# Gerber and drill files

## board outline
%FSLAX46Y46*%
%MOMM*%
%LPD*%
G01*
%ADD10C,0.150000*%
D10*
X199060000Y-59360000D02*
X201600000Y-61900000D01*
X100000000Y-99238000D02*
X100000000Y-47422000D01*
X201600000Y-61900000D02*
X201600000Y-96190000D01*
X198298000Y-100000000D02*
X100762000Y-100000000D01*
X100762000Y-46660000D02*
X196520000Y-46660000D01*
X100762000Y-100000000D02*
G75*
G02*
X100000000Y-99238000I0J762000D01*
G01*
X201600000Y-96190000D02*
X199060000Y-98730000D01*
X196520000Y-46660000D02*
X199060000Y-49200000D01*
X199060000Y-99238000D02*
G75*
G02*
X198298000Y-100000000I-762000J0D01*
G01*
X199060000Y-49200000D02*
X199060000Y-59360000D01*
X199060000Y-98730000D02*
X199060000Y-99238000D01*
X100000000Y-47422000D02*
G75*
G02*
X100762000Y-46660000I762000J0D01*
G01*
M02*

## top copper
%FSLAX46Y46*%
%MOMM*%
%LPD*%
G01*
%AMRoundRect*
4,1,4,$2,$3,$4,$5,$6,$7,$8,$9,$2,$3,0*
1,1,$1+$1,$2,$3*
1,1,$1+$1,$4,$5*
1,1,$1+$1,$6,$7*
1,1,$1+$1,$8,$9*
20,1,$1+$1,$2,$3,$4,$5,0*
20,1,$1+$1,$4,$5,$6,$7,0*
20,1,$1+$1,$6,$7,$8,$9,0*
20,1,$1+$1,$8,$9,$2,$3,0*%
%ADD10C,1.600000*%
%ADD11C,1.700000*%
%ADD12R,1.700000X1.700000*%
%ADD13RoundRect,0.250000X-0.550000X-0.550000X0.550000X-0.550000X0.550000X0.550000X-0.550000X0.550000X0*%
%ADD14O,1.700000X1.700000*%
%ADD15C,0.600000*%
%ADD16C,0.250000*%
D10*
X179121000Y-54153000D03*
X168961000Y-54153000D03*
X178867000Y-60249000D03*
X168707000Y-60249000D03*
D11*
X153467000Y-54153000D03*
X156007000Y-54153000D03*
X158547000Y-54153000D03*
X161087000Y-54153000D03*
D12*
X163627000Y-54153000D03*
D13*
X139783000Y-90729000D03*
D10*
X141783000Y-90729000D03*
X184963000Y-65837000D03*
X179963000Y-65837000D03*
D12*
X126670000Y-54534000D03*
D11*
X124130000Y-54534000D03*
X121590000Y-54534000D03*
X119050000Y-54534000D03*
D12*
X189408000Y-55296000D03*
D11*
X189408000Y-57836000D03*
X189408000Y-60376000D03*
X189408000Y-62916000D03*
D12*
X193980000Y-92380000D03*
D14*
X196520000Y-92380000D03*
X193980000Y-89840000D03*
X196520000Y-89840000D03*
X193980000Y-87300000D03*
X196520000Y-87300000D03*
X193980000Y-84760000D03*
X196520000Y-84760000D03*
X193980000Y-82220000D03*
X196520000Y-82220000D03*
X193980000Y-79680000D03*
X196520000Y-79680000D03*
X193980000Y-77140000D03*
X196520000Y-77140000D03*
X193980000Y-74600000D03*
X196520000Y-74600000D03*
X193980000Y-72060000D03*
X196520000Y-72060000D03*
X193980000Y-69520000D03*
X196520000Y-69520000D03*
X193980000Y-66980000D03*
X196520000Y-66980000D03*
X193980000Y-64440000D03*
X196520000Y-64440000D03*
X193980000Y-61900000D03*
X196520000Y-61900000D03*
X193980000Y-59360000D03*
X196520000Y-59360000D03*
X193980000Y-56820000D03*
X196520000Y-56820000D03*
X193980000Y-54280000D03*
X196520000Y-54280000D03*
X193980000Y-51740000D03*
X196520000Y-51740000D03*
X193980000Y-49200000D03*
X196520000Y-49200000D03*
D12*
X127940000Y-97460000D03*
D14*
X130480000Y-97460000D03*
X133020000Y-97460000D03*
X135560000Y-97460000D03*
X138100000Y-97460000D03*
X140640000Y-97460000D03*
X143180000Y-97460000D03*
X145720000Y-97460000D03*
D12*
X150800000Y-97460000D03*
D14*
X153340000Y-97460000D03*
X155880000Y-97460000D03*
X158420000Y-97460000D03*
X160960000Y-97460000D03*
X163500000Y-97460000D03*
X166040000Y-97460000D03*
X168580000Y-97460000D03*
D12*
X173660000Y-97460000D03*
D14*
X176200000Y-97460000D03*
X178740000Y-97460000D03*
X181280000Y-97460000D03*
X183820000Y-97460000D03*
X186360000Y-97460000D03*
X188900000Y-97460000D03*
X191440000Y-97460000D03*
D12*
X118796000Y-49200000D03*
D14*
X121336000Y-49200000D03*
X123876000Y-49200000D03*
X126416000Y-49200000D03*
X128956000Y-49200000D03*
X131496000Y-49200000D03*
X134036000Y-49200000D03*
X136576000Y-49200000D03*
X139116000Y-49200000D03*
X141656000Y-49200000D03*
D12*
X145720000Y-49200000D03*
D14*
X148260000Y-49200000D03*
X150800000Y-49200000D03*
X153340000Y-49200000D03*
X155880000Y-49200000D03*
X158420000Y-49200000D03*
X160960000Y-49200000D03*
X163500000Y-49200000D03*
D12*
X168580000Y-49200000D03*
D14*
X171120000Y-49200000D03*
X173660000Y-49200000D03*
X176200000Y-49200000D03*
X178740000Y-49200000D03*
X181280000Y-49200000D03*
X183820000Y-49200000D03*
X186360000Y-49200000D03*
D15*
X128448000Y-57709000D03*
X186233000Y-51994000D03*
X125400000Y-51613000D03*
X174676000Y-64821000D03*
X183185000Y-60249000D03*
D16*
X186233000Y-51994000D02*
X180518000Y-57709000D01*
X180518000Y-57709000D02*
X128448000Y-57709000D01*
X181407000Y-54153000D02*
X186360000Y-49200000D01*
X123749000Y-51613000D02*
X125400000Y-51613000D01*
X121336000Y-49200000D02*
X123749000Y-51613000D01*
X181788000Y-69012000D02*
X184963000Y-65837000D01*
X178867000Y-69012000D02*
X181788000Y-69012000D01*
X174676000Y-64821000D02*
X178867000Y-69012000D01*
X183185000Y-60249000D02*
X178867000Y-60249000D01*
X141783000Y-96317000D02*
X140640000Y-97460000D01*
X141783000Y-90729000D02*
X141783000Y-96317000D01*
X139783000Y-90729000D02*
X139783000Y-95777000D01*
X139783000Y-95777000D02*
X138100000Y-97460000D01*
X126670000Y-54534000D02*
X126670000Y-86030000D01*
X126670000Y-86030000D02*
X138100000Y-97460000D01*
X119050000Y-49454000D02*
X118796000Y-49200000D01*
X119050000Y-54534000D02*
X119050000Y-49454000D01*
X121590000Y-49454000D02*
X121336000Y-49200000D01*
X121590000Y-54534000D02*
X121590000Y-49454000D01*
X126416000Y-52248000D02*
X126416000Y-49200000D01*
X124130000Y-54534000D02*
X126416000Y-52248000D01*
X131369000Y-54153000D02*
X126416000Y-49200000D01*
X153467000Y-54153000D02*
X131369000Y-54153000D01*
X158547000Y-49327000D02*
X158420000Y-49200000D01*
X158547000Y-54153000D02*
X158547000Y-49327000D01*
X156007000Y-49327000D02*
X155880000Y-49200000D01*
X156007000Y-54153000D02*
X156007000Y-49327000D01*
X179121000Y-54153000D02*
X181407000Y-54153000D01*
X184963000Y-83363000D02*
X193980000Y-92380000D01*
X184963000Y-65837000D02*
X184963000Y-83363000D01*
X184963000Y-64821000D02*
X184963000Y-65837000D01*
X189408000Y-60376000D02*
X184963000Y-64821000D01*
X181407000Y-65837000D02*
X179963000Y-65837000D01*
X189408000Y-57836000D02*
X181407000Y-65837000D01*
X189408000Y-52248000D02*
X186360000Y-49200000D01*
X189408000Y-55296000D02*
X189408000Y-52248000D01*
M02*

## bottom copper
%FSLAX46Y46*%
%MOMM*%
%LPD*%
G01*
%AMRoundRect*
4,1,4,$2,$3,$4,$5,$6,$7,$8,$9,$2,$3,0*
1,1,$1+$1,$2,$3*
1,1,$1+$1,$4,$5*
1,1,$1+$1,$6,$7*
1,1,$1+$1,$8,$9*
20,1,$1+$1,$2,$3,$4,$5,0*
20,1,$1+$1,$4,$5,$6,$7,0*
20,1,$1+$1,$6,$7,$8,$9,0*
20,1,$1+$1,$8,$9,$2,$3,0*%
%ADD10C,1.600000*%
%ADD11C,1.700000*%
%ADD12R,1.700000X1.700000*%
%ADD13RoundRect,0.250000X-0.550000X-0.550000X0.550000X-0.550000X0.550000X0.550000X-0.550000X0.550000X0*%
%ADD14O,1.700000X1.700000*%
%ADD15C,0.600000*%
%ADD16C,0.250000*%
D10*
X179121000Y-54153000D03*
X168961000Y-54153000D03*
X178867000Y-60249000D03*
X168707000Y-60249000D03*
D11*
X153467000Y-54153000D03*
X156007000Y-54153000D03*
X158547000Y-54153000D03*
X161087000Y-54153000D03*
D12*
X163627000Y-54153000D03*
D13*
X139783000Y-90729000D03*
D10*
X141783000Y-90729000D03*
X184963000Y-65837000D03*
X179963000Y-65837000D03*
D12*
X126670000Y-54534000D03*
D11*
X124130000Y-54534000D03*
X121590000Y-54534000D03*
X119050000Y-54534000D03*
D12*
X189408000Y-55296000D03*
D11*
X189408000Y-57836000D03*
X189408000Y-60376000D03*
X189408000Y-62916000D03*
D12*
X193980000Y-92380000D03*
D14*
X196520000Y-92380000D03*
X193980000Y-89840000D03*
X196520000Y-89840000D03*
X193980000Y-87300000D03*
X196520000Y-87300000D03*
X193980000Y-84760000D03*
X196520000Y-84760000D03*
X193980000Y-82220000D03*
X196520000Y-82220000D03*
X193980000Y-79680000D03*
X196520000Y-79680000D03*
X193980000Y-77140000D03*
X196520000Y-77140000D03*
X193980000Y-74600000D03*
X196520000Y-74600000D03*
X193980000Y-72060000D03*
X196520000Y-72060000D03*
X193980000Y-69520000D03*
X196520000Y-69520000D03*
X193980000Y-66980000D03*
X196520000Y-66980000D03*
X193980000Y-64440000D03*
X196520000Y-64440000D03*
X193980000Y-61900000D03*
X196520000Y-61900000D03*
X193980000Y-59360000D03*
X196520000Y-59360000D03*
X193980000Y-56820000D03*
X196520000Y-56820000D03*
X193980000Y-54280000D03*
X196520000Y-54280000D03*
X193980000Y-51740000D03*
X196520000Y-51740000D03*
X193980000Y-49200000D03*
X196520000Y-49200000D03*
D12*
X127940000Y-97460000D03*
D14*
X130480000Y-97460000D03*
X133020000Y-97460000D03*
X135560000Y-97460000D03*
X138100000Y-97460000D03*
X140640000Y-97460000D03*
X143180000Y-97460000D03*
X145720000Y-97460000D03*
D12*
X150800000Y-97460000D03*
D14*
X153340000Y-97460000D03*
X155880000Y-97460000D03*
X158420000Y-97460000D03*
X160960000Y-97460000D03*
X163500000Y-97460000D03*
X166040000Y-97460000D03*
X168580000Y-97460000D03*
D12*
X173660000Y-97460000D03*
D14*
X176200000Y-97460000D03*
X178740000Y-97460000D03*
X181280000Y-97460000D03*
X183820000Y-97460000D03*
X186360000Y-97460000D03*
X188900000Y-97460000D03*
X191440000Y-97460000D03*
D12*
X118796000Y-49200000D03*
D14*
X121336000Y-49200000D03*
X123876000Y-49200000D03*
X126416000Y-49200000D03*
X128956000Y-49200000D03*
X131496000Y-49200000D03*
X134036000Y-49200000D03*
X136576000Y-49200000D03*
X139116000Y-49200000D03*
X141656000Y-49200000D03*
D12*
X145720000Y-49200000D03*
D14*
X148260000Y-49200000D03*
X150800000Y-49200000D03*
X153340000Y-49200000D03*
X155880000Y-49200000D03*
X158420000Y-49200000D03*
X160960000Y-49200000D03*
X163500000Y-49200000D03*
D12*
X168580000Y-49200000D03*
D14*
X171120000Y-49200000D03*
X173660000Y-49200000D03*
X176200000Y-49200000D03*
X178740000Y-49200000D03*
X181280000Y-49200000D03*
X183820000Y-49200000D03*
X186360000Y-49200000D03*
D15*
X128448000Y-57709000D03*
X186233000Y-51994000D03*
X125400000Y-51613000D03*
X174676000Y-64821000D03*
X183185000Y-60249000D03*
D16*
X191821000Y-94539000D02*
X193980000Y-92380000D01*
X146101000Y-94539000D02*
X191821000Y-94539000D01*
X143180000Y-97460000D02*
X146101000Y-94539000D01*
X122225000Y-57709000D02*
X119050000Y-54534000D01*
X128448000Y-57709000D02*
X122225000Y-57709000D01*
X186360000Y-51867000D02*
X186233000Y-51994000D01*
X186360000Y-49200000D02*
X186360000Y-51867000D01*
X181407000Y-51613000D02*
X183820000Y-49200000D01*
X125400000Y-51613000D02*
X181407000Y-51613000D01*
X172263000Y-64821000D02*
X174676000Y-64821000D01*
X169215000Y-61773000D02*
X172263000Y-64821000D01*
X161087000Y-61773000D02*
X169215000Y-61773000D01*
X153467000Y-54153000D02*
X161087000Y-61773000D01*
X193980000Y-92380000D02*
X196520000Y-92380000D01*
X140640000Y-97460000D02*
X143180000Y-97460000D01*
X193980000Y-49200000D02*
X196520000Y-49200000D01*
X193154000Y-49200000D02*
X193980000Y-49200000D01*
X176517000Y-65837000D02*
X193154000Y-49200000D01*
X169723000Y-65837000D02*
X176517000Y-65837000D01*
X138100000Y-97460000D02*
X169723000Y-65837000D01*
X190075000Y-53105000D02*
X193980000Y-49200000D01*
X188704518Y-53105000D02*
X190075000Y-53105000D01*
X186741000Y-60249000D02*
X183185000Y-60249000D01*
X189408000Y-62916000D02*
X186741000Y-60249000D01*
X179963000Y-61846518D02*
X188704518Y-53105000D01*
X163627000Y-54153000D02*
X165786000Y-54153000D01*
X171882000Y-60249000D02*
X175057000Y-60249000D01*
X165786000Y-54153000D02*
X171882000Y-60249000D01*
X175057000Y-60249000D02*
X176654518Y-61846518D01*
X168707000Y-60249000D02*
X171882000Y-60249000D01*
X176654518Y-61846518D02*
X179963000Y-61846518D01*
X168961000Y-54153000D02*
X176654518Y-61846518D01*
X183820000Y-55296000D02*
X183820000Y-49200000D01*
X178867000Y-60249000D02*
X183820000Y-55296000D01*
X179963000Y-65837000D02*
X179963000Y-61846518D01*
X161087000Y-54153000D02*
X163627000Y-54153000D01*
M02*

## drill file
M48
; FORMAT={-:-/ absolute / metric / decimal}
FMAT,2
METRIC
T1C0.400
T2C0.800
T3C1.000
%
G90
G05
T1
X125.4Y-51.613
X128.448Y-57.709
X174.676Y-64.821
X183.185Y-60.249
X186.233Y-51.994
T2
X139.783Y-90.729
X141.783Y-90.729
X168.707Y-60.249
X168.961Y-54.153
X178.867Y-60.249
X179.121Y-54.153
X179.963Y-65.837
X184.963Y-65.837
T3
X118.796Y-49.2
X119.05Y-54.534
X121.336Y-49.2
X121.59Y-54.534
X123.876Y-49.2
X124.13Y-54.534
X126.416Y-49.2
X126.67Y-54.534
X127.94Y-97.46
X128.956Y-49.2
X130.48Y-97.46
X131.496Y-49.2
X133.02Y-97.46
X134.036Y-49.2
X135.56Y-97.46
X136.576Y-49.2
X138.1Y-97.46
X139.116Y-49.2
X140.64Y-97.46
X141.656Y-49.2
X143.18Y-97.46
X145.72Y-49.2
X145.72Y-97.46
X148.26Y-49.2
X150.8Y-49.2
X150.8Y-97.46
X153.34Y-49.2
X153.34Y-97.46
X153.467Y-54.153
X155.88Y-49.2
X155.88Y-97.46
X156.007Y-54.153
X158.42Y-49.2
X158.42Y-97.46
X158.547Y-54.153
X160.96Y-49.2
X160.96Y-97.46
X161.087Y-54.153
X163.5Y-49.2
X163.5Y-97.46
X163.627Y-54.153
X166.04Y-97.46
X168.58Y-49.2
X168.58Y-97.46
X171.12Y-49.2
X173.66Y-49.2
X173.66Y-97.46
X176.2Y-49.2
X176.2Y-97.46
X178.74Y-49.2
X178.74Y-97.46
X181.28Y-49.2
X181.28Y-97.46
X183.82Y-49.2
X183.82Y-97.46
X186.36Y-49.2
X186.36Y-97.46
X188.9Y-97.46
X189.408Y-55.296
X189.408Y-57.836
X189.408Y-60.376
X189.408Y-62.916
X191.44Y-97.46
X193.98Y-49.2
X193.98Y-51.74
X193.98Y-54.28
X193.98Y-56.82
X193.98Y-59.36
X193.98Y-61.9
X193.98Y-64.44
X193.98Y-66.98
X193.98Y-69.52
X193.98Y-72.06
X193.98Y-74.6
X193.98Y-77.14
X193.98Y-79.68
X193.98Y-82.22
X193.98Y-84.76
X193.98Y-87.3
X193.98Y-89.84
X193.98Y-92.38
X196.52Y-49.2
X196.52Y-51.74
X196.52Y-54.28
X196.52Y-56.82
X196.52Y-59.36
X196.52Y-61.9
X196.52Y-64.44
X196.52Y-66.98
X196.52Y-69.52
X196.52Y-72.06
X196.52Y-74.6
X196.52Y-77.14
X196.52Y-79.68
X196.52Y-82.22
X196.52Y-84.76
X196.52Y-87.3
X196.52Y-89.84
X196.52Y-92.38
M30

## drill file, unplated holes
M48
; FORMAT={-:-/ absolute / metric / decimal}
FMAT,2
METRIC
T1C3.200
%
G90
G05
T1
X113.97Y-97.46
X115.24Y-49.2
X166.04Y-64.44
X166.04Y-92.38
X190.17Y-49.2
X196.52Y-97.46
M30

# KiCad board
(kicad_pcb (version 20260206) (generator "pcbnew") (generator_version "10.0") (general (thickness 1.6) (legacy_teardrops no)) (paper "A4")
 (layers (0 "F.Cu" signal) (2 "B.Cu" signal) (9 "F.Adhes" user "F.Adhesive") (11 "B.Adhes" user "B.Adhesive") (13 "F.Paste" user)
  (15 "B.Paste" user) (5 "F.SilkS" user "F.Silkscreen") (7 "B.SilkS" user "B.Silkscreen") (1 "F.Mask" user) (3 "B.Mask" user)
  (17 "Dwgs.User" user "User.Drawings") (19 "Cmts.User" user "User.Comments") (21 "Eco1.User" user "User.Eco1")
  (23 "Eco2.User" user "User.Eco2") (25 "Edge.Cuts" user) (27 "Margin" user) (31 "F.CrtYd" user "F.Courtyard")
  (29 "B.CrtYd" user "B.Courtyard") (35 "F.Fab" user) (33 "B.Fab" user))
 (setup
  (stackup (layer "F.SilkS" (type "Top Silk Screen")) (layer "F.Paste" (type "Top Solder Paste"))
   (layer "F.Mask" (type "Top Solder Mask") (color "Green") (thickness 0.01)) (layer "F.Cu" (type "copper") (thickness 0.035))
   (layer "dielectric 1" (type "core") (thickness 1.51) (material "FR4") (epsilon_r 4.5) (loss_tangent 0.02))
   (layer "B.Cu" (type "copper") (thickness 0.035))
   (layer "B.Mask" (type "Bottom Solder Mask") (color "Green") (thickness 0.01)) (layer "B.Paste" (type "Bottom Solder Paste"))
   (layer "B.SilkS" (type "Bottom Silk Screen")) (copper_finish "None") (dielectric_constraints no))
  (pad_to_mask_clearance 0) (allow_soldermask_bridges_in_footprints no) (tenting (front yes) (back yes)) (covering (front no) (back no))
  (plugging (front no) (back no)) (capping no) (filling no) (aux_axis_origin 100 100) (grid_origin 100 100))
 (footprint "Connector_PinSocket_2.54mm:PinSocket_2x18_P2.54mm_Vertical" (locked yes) (layer "F.Cu") (at 193.98 92.38 180)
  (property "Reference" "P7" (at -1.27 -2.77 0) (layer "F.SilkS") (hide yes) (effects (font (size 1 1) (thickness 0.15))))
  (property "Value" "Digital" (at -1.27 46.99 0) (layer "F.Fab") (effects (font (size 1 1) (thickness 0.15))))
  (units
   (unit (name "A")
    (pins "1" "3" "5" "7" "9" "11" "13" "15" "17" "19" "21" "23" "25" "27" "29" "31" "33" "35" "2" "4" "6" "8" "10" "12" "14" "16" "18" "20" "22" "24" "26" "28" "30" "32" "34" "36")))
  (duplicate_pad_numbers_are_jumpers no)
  (pad "1" thru_hole rect (at 0 0 180) (size 1.7 1.7) (drill 1) (layers "*.Cu" "*.Mask") (remove_unused_layers no) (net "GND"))
  (pad "2" thru_hole oval (at -2.54 0 180) (size 1.7 1.7) (drill 1) (layers "*.Cu" "*.Mask") (remove_unused_layers no) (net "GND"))
  (pad "3" thru_hole oval (at 0 2.54 180) (size 1.7 1.7) (drill 1) (layers "*.Cu" "*.Mask") (remove_unused_layers no) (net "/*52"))
  (pad "4" thru_hole oval (at -2.54 2.54 180) (size 1.7 1.7) (drill 1) (layers "*.Cu" "*.Mask") (remove_unused_layers no) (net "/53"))
  (pad "5" thru_hole oval (at 0 5.08 180) (size 1.7 1.7) (drill 1) (layers "*.Cu" "*.Mask") (remove_unused_layers no) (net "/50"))
  (pad "6" thru_hole oval (at -2.54 5.08 180) (size 1.7 1.7) (drill 1) (layers "*.Cu" "*.Mask") (remove_unused_layers no) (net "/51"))
  (pad "7" thru_hole oval (at 0 7.62 180) (size 1.7 1.7) (drill 1) (layers "*.Cu" "*.Mask") (remove_unused_layers no) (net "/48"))
  (pad "8" thru_hole oval (at -2.54 7.62 180) (size 1.7 1.7) (drill 1) (layers "*.Cu" "*.Mask") (remove_unused_layers no) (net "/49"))
  (pad "9" thru_hole oval (at 0 10.16 180) (size 1.7 1.7) (drill 1) (layers "*.Cu" "*.Mask") (remove_unused_layers no) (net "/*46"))
  (pad "10" thru_hole oval (at -2.54 10.16 180) (size 1.7 1.7) (drill 1) (layers "*.Cu" "*.Mask") (remove_unused_layers no) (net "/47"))
  (pad "11" thru_hole oval (at 0 12.7 180) (size 1.7 1.7) (drill 1) (layers "*.Cu" "*.Mask") (remove_unused_layers no) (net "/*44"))
  (pad "12" thru_hole oval (at -2.54 12.7 180) (size 1.7 1.7) (drill 1) (layers "*.Cu" "*.Mask") (remove_unused_layers no) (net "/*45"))
  (pad "13" thru_hole oval (at 0 15.24 180) (size 1.7 1.7) (drill 1) (layers "*.Cu" "*.Mask") (remove_unused_layers no) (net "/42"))
  (pad "14" thru_hole oval (at -2.54 15.24 180) (size 1.7 1.7) (drill 1) (layers "*.Cu" "*.Mask") (remove_unused_layers no) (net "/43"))
  (pad "15" thru_hole oval (at 0 17.78 180) (size 1.7 1.7) (drill 1) (layers "*.Cu" "*.Mask") (remove_unused_layers no) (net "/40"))
  (pad "16" thru_hole oval (at -2.54 17.78 180) (size 1.7 1.7) (drill 1) (layers "*.Cu" "*.Mask") (remove_unused_layers no) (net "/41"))
  (pad "17" thru_hole oval (at 0 20.32 180) (size 1.7 1.7) (drill 1) (layers "*.Cu" "*.Mask") (remove_unused_layers no) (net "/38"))
  (pad "18" thru_hole oval (at -2.54 20.32 180) (size 1.7 1.7) (drill 1) (layers "*.Cu" "*.Mask") (remove_unused_layers no) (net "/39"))
  (pad "19" thru_hole oval (at 0 22.86 180) (size 1.7 1.7) (drill 1) (layers "*.Cu" "*.Mask") (remove_unused_layers no) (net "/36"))
  (pad "20" thru_hole oval (at -2.54 22.86 180) (size 1.7 1.7) (drill 1) (layers "*.Cu" "*.Mask") (remove_unused_layers no) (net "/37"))
  (pad "21" thru_hole oval (at 0 25.4 180) (size 1.7 1.7) (drill 1) (layers "*.Cu" "*.Mask") (remove_unused_layers no) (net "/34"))
  (pad "22" thru_hole oval (at -2.54 25.4 180) (size 1.7 1.7) (drill 1) (layers "*.Cu" "*.Mask") (remove_unused_layers no) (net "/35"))
  (pad "23" thru_hole oval (at 0 27.94 180) (size 1.7 1.7) (drill 1) (layers "*.Cu" "*.Mask") (remove_unused_layers no) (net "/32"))
  (pad "24" thru_hole oval (at -2.54 27.94 180) (size 1.7 1.7) (drill 1) (layers "*.Cu" "*.Mask") (remove_unused_layers no) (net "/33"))
  (pad "25" thru_hole oval (at 0 30.48 180) (size 1.7 1.7) (drill 1) (layers "*.Cu" "*.Mask") (remove_unused_layers no) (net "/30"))
  (pad "26" thru_hole oval (at -2.54 30.48 180) (size 1.7 1.7) (drill 1) (layers "*.Cu" "*.Mask") (remove_unused_layers no) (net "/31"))
  (pad "27" thru_hole oval (at 0 33.02 180) (size 1.7 1.7) (drill 1) (layers "*.Cu" "*.Mask") (remove_unused_layers no) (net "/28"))
  (pad "28" thru_hole oval (at -2.54 33.02 180) (size 1.7 1.7) (drill 1) (layers "*.Cu" "*.Mask") (remove_unused_layers no) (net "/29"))
  (pad "29" thru_hole oval (at 0 35.56 180) (size 1.7 1.7) (drill 1) (layers "*.Cu" "*.Mask") (remove_unused_layers no) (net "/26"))
  (pad "30" thru_hole oval (at -2.54 35.56 180) (size 1.7 1.7) (drill 1) (layers "*.Cu" "*.Mask") (remove_unused_layers no) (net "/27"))
  (pad "31" thru_hole oval (at 0 38.1 180) (size 1.7 1.7) (drill 1) (layers "*.Cu" "*.Mask") (remove_unused_layers no) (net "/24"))
  (pad "32" thru_hole oval (at -2.54 38.1 180) (size 1.7 1.7) (drill 1) (layers "*.Cu" "*.Mask") (remove_unused_layers no) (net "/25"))
  (pad "33" thru_hole oval (at 0 40.64 180) (size 1.7 1.7) (drill 1) (layers "*.Cu" "*.Mask") (remove_unused_layers no) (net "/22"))
  (pad "34" thru_hole oval (at -2.54 40.64 180) (size 1.7 1.7) (drill 1) (layers "*.Cu" "*.Mask") (remove_unused_layers no) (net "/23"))
  (pad "35" thru_hole oval (at 0 43.18 180) (size 1.7 1.7) (drill 1) (layers "*.Cu" "*.Mask") (remove_unused_layers no) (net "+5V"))
  (pad "36" thru_hole oval (at -2.54 43.18 180) (size 1.7 1.7) (drill 1) (layers "*.Cu" "*.Mask") (remove_unused_layers no) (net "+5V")))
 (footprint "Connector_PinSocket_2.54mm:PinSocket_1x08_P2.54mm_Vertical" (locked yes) (layer "F.Cu") (at 127.94 97.46 90)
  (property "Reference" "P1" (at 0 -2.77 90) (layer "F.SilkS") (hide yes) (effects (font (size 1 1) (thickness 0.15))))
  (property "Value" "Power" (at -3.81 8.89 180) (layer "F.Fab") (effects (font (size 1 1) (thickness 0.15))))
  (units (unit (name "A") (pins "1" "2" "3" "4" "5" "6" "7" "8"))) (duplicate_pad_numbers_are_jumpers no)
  (pad "1" thru_hole rect (at 0 0 90) (size 1.7 1.7) (drill 1) (layers "*.Cu" "*.Mask") (remove_unused_layers no)
   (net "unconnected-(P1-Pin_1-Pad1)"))
  (pad "2" thru_hole oval (at 0 2.54 90) (size 1.7 1.7) (drill 1) (layers "*.Cu" "*.Mask") (remove_unused_layers no) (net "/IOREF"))
  (pad "3" thru_hole oval (at 0 5.08 90) (size 1.7 1.7) (drill 1) (layers "*.Cu" "*.Mask") (remove_unused_layers no) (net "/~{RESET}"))
  (pad "4" thru_hole oval (at 0 7.62 90) (size 1.7 1.7) (drill 1) (layers "*.Cu" "*.Mask") (remove_unused_layers no) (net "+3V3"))
  (pad "5" thru_hole oval (at 0 10.16 90) (size 1.7 1.7) (drill 1) (layers "*.Cu" "*.Mask") (remove_unused_layers no) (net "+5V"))
  (pad "6" thru_hole oval (at 0 12.7 90) (size 1.7 1.7) (drill 1) (layers "*.Cu" "*.Mask") (remove_unused_layers no) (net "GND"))
  (pad "7" thru_hole oval (at 0 15.24 90) (size 1.7 1.7) (drill 1) (layers "*.Cu" "*.Mask") (remove_unused_layers no) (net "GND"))
  (pad "8" thru_hole oval (at 0 17.78 90) (size 1.7 1.7) (drill 1) (layers "*.Cu" "*.Mask") (remove_unused_layers no) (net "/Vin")))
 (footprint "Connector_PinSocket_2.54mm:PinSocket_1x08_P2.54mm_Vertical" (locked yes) (layer "F.Cu") (at 150.8 97.46 90)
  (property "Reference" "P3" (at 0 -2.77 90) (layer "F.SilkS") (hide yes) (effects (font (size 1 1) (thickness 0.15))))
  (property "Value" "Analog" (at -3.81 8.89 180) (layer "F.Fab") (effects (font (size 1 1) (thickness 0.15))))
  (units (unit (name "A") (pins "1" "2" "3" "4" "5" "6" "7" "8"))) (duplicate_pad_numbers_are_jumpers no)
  (pad "1" thru_hole rect (at 0 0 90) (size 1.7 1.7) (drill 1) (layers "*.Cu" "*.Mask") (remove_unused_layers no) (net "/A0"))
  (pad "2" thru_hole oval (at 0 2.54 90) (size 1.7 1.7) (drill 1) (layers "*.Cu" "*.Mask") (remove_unused_layers no) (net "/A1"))
  (pad "3" thru_hole oval (at 0 5.08 90) (size 1.7 1.7) (drill 1) (layers "*.Cu" "*.Mask") (remove_unused_layers no) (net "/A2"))
  (pad "4" thru_hole oval (at 0 7.62 90) (size 1.7 1.7) (drill 1) (layers "*.Cu" "*.Mask") (remove_unused_layers no) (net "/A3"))
  (pad "5" thru_hole oval (at 0 10.16 90) (size 1.7 1.7) (drill 1) (layers "*.Cu" "*.Mask") (remove_unused_layers no) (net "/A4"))
  (pad "6" thru_hole oval (at 0 12.7 90) (size 1.7 1.7) (drill 1) (layers "*.Cu" "*.Mask") (remove_unused_layers no) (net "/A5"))
  (pad "7" thru_hole oval (at 0 15.24 90) (size 1.7 1.7) (drill 1) (layers "*.Cu" "*.Mask") (remove_unused_layers no) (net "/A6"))
  (pad "8" thru_hole oval (at 0 17.78 90) (size 1.7 1.7) (drill 1) (layers "*.Cu" "*.Mask") (remove_unused_layers no) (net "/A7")))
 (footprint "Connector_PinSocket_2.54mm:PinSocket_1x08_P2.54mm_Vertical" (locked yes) (layer "F.Cu") (at 173.66 97.46 90)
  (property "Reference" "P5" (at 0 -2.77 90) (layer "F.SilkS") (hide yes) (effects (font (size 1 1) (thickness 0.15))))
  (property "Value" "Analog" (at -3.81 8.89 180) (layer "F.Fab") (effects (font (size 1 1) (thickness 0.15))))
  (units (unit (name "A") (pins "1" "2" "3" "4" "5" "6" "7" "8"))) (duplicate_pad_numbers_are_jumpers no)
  (pad "1" thru_hole rect (at 0 0 90) (size 1.7 1.7) (drill 1) (layers "*.Cu" "*.Mask") (remove_unused_layers no) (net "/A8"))
  (pad "2" thru_hole oval (at 0 2.54 90) (size 1.7 1.7) (drill 1) (layers "*.Cu" "*.Mask") (remove_unused_layers no) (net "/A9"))
  (pad "3" thru_hole oval (at 0 5.08 90) (size 1.7 1.7) (drill 1) (layers "*.Cu" "*.Mask") (remove_unused_layers no) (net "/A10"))
  (pad "4" thru_hole oval (at 0 7.62 90) (size 1.7 1.7) (drill 1) (layers "*.Cu" "*.Mask") (remove_unused_layers no) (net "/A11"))
  (pad "5" thru_hole oval (at 0 10.16 90) (size 1.7 1.7) (drill 1) (layers "*.Cu" "*.Mask") (remove_unused_layers no) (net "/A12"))
  (pad "6" thru_hole oval (at 0 12.7 90) (size 1.7 1.7) (drill 1) (layers "*.Cu" "*.Mask") (remove_unused_layers no) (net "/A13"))
  (pad "7" thru_hole oval (at 0 15.24 90) (size 1.7 1.7) (drill 1) (layers "*.Cu" "*.Mask") (remove_unused_layers no) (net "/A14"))
  (pad "8" thru_hole oval (at 0 17.78 90) (size 1.7 1.7) (drill 1) (layers "*.Cu" "*.Mask") (remove_unused_layers no) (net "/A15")))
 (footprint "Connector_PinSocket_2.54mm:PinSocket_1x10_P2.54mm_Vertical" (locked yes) (layer "F.Cu") (at 118.796 49.2 90)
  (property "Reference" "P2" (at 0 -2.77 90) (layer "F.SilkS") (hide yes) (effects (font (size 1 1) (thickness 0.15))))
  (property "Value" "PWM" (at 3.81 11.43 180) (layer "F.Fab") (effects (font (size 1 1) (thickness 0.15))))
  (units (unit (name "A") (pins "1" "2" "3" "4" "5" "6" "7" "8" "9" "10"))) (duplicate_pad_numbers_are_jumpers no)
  (pad "1" thru_hole rect (at 0 0 90) (size 1.7 1.7) (drill 1) (layers "*.Cu" "*.Mask") (remove_unused_layers no) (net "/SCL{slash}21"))
  (pad "2" thru_hole oval (at 0 2.54 90) (size 1.7 1.7) (drill 1) (layers "*.Cu" "*.Mask") (remove_unused_layers no) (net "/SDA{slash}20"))
  (pad "3" thru_hole oval (at 0 5.08 90) (size 1.7 1.7) (drill 1) (layers "*.Cu" "*.Mask") (remove_unused_layers no) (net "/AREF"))
  (pad "4" thru_hole oval (at 0 7.62 90) (size 1.7 1.7) (drill 1) (layers "*.Cu" "*.Mask") (remove_unused_layers no) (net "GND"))
  (pad "5" thru_hole oval (at 0 10.16 90) (size 1.7 1.7) (drill 1) (layers "*.Cu" "*.Mask") (remove_unused_layers no) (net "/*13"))
  (pad "6" thru_hole oval (at 0 12.7 90) (size 1.7 1.7) (drill 1) (layers "*.Cu" "*.Mask") (remove_unused_layers no) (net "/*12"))
  (pad "7" thru_hole oval (at 0 15.24 90) (size 1.7 1.7) (drill 1) (layers "*.Cu" "*.Mask") (remove_unused_layers no) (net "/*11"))
  (pad "8" thru_hole oval (at 0 17.78 90) (size 1.7 1.7) (drill 1) (layers "*.Cu" "*.Mask") (remove_unused_layers no) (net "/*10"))
  (pad "9" thru_hole oval (at 0 20.32 90) (size 1.7 1.7) (drill 1) (layers "*.Cu" "*.Mask") (remove_unused_layers no) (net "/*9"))
  (pad "10" thru_hole oval (at 0 22.86 90) (size 1.7 1.7) (drill 1) (layers "*.Cu" "*.Mask") (remove_unused_layers no) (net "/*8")))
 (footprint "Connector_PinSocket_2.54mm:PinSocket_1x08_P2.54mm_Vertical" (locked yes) (layer "F.Cu") (at 145.72 49.2 90)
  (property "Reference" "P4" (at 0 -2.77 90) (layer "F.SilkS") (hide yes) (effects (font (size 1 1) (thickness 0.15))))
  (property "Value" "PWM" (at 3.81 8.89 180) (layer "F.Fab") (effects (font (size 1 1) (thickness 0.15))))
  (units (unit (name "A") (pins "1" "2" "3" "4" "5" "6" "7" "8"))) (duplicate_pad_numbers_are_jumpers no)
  (pad "1" thru_hole rect (at 0 0 90) (size 1.7 1.7) (drill 1) (layers "*.Cu" "*.Mask") (remove_unused_layers no) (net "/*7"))
  (pad "2" thru_hole oval (at 0 2.54 90) (size 1.7 1.7) (drill 1) (layers "*.Cu" "*.Mask") (remove_unused_layers no) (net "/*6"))
  (pad "3" thru_hole oval (at 0 5.08 90) (size 1.7 1.7) (drill 1) (layers "*.Cu" "*.Mask") (remove_unused_layers no) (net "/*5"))
  (pad "4" thru_hole oval (at 0 7.62 90) (size 1.7 1.7) (drill 1) (layers "*.Cu" "*.Mask") (remove_unused_layers no) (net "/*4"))
  (pad "5" thru_hole oval (at 0 10.16 90) (size 1.7 1.7) (drill 1) (layers "*.Cu" "*.Mask") (remove_unused_layers no) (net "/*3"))
  (pad "6" thru_hole oval (at 0 12.7 90) (size 1.7 1.7) (drill 1) (layers "*.Cu" "*.Mask") (remove_unused_layers no) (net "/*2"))
  (pad "7" thru_hole oval (at 0 15.24 90) (size 1.7 1.7) (drill 1) (layers "*.Cu" "*.Mask") (remove_unused_layers no) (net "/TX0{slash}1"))
  (pad "8" thru_hole oval (at 0 17.78 90) (size 1.7 1.7) (drill 1) (layers "*.Cu" "*.Mask") (remove_unused_layers no) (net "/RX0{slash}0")))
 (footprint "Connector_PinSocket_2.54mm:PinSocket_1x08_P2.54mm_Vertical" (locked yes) (layer "F.Cu") (at 168.58 49.2 90)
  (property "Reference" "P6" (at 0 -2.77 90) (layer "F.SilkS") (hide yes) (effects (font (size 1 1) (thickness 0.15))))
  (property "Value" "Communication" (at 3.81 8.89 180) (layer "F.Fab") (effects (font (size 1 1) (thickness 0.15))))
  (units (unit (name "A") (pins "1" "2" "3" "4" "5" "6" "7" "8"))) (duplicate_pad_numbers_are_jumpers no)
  (pad "1" thru_hole rect (at 0 0 90) (size 1.7 1.7) (drill 1) (layers "*.Cu" "*.Mask") (remove_unused_layers no) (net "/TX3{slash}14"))
  (pad "2" thru_hole oval (at 0 2.54 90) (size 1.7 1.7) (drill 1) (layers "*.Cu" "*.Mask") (remove_unused_layers no) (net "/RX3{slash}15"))
  (pad "3" thru_hole oval (at 0 5.08 90) (size 1.7 1.7) (drill 1) (layers "*.Cu" "*.Mask") (remove_unused_layers no) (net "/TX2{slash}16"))
  (pad "4" thru_hole oval (at 0 7.62 90) (size 1.7 1.7) (drill 1) (layers "*.Cu" "*.Mask") (remove_unused_layers no) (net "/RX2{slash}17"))
  (pad "5" thru_hole oval (at 0 10.16 90) (size 1.7 1.7) (drill 1) (layers "*.Cu" "*.Mask") (remove_unused_layers no) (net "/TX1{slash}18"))
  (pad "6" thru_hole oval (at 0 12.7 90) (size 1.7 1.7) (drill 1) (layers "*.Cu" "*.Mask") (remove_unused_layers no) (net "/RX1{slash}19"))
  (pad "7" thru_hole oval (at 0 15.24 90) (size 1.7 1.7) (drill 1) (layers "*.Cu" "*.Mask") (remove_unused_layers no) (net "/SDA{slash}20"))
  (pad "8" thru_hole oval (at 0 17.78 90) (size 1.7 1.7) (drill 1) (layers "*.Cu" "*.Mask") (remove_unused_layers no) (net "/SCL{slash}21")))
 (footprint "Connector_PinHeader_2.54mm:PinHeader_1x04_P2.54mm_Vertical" (layer "F.Cu") (at 189.408 55.296)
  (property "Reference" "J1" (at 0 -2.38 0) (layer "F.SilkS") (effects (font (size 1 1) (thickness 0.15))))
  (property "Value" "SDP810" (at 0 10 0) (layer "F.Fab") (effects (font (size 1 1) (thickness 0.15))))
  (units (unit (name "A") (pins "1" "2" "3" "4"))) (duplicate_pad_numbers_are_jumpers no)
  (pad "1" thru_hole rect (at 0 0) (size 1.7 1.7) (drill 1) (layers "*.Cu" "*.Mask") (remove_unused_layers no) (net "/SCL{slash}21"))
  (pad "2" thru_hole circle (at 0 2.54) (size 1.7 1.7) (drill 1) (layers "*.Cu" "*.Mask") (remove_unused_layers no) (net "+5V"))
  (pad "3" thru_hole circle (at 0 5.08) (size 1.7 1.7) (drill 1) (layers "*.Cu" "*.Mask") (remove_unused_layers no) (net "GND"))
  (pad "4" thru_hole circle (at 0 7.62) (size 1.7 1.7) (drill 1) (layers "*.Cu" "*.Mask") (remove_unused_layers no) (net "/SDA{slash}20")))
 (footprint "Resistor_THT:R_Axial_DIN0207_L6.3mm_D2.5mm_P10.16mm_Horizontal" (layer "F.Cu") (at 168.961 54.153)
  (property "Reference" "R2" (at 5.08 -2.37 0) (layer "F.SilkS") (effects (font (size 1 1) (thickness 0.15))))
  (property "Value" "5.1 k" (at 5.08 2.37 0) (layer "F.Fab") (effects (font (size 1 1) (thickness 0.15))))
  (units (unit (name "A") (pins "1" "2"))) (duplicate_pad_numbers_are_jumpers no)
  (pad "1" thru_hole circle (at 0 0) (size 1.6 1.6) (drill 0.8) (layers "*.Cu" "*.Mask") (remove_unused_layers no) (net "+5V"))
  (pad "2" thru_hole circle (at 10.16 0) (size 1.6 1.6) (drill 0.8) (layers "*.Cu" "*.Mask") (remove_unused_layers no) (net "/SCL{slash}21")))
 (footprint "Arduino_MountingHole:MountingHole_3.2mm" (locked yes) (layer "F.Cu") (at 196.52 97.46)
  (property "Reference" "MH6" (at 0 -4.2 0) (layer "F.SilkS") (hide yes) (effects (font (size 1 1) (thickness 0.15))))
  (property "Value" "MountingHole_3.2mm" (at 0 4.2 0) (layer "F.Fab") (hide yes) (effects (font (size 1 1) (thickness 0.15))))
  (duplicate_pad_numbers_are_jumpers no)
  (pad "" np_thru_hole circle (at 0 0) (size 3.2 3.2) (drill 3.2) (layers "*.Cu" "*.Mask")))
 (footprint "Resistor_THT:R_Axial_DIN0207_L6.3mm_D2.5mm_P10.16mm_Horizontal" (layer "F.Cu") (at 168.707 60.249)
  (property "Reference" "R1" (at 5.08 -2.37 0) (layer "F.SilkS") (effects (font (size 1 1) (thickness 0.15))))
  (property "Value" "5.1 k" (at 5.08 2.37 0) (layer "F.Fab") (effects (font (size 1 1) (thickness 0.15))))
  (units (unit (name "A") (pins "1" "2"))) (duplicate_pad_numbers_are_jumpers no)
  (pad "1" thru_hole circle (at 0 0) (size 1.6 1.6) (drill 0.8) (layers "*.Cu" "*.Mask") (remove_unused_layers no) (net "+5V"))
  (pad "2" thru_hole circle (at 10.16 0) (size 1.6 1.6) (drill 0.8) (layers "*.Cu" "*.Mask") (remove_unused_layers no) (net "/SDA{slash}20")))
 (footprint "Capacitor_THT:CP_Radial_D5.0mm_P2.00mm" (layer "F.Cu") (at 139.783 90.729)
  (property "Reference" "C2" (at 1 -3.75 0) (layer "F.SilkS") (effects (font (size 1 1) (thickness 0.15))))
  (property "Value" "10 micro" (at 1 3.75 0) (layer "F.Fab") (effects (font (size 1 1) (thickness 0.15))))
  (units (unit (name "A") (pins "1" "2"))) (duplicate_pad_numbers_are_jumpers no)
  (pad "1" thru_hole roundrect (at 0 0) (size 1.6 1.6) (drill 0.8) (layers "*.Cu" "*.Mask") (remove_unused_layers no)
   (roundrect_rratio 0.15625) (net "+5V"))
  (pad "2" thru_hole circle (at 2 0) (size 1.6 1.6) (drill 0.8) (layers "*.Cu" "*.Mask") (remove_unused_layers no) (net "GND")))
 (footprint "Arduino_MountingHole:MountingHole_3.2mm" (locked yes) (layer "F.Cu") (at 115.24 49.2)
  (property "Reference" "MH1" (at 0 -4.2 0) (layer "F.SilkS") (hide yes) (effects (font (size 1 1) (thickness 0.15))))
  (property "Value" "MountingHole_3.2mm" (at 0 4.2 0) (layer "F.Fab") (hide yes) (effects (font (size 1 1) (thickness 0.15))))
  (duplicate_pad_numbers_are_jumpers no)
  (pad "" np_thru_hole circle (at 0 0) (size 3.2 3.2) (drill 3.2) (layers "*.Cu" "*.Mask")))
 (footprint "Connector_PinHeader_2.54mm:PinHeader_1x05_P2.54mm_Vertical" (layer "F.Cu") (at 163.627 54.153 -90)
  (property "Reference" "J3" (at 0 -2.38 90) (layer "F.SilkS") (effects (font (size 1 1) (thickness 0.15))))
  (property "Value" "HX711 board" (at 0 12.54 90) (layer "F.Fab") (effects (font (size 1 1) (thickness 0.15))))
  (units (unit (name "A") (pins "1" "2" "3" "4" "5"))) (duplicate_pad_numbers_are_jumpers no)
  (pad "1" thru_hole rect (at 0 0 270) (size 1.7 1.7) (drill 1) (layers "*.Cu" "*.Mask") (remove_unused_layers no) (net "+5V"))
  (pad "2" thru_hole circle (at 0 2.54 270) (size 1.7 1.7) (drill 1) (layers "*.Cu" "*.Mask") (remove_unused_layers no) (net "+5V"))
  (pad "3" thru_hole circle (at 0 5.08 270) (size 1.7 1.7) (drill 1) (layers "*.Cu" "*.Mask") (remove_unused_layers no) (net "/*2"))
  (pad "4" thru_hole circle (at 0 7.62 270) (size 1.7 1.7) (drill 1) (layers "*.Cu" "*.Mask") (remove_unused_layers no) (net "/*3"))
  (pad "5" thru_hole circle (at 0 10.16 270) (size 1.7 1.7) (drill 1) (layers "*.Cu" "*.Mask") (remove_unused_layers no) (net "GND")))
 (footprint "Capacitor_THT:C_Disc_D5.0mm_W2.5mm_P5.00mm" (layer "F.Cu") (at 179.963 65.837)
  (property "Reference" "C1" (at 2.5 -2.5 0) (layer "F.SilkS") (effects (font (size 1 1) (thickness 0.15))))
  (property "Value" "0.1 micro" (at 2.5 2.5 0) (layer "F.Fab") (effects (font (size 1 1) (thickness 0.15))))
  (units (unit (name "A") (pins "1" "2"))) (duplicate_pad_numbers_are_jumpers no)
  (pad "1" thru_hole circle (at 0 0) (size 1.6 1.6) (drill 0.8) (layers "*.Cu" "*.Mask") (remove_unused_layers no) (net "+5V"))
  (pad "2" thru_hole circle (at 5 0) (size 1.6 1.6) (drill 0.8) (layers "*.Cu" "*.Mask") (remove_unused_layers no) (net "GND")))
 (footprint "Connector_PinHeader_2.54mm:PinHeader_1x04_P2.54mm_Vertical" (layer "F.Cu") (at 126.67 54.534 -90)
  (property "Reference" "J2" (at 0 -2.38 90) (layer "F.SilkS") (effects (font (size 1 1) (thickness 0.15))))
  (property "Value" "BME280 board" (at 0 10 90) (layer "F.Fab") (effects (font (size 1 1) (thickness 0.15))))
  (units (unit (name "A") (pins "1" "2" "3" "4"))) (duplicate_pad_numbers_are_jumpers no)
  (pad "1" thru_hole rect (at 0 0 270) (size 1.7 1.7) (drill 1) (layers "*.Cu" "*.Mask") (remove_unused_layers no) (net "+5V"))
  (pad "2" thru_hole circle (at 0 2.54 270) (size 1.7 1.7) (drill 1) (layers "*.Cu" "*.Mask") (remove_unused_layers no) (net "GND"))
  (pad "3" thru_hole circle (at 0 5.08 270) (size 1.7 1.7) (drill 1) (layers "*.Cu" "*.Mask") (remove_unused_layers no)
   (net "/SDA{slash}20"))
  (pad "4" thru_hole circle (at 0 7.62 270) (size 1.7 1.7) (drill 1) (layers "*.Cu" "*.Mask") (remove_unused_layers no)
   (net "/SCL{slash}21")))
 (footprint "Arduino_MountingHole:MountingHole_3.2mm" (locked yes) (layer "F.Cu") (at 113.97 97.46)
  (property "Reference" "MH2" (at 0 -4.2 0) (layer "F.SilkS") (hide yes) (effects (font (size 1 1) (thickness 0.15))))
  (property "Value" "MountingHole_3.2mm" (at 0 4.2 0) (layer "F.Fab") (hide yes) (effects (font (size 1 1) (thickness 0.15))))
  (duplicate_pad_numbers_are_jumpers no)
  (pad "" np_thru_hole circle (at 0 0) (size 3.2 3.2) (drill 3.2) (layers "*.Cu" "*.Mask")))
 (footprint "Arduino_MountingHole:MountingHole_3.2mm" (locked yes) (layer "F.Cu") (at 166.04 64.44)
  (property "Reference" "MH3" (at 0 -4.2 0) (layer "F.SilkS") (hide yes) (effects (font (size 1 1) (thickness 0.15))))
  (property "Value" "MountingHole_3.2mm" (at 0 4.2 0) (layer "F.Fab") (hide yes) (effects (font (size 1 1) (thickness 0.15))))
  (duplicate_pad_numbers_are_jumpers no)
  (pad "" np_thru_hole circle (at 0 0) (size 3.2 3.2) (drill 3.2) (layers "*.Cu" "*.Mask")))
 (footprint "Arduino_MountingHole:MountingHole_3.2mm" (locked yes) (layer "F.Cu") (at 166.04 92.38)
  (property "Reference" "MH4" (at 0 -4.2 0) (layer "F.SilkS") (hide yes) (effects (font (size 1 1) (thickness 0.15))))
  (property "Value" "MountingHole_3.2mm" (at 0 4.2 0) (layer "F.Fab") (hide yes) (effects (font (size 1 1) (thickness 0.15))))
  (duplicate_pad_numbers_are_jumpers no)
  (pad "" np_thru_hole circle (at 0 0) (size 3.2 3.2) (drill 3.2) (layers "*.Cu" "*.Mask")))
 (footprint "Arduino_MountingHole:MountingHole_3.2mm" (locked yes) (layer "F.Cu") (at 190.17 49.2)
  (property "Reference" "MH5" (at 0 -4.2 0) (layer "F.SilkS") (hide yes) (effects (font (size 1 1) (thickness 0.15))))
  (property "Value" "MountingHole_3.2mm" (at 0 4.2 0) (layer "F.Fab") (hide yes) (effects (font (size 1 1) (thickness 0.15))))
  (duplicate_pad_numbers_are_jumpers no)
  (pad "" np_thru_hole circle (at 0 0) (size 3.2 3.2) (drill 3.2) (layers "*.Cu" "*.Mask")))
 (gr_arc (start 100 47.422) (mid 100.223185 46.883185) (end 100.762 46.66) (stroke (width 0.15) (type solid)) (layer "Edge.Cuts"))
 (gr_line (start 100 99.238) (end 100 47.422) (stroke (width 0.15) (type solid)) (layer "Edge.Cuts"))
 (gr_line (start 100.762 46.66) (end 196.52 46.66) (stroke (width 0.15) (type solid)) (layer "Edge.Cuts"))
 (gr_arc (start 100.762 100) (mid 100.223185 99.776815) (end 100 99.238) (stroke (width 0.15) (type solid)) (layer "Edge.Cuts"))
 (gr_line (start 196.52 46.66) (end 199.06 49.2) (stroke (width 0.15) (type solid)) (layer "Edge.Cuts"))
 (gr_line (start 198.298 100) (end 100.762 100) (stroke (width 0.15) (type solid)) (layer "Edge.Cuts"))
 (gr_line (start 199.06 49.2) (end 199.06 59.36) (stroke (width 0.15) (type solid)) (layer "Edge.Cuts"))
 (gr_line (start 199.06 59.36) (end 201.6 61.9) (stroke (width 0.15) (type solid)) (layer "Edge.Cuts"))
 (gr_line (start 199.06 98.73) (end 199.06 99.238) (stroke (width 0.15) (type solid)) (layer "Edge.Cuts"))
 (gr_arc (start 199.06 99.238) (mid 198.836815 99.776815) (end 198.298 100) (stroke (width 0.15) (type solid)) (layer "Edge.Cuts"))
 (gr_line (start 201.6 61.9) (end 201.6 96.19) (stroke (width 0.15) (type solid)) (layer "Edge.Cuts"))
 (gr_line (start 201.6 96.19) (end 199.06 98.73) (stroke (width 0.15) (type solid)) (layer "Edge.Cuts"))
 (segment (start 124.13 54.534) (end 126.416 52.248) (width 0.25) (layer "F.Cu") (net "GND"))
 (segment (start 153.467 54.153) (end 131.369 54.153) (width 0.25) (layer "F.Cu") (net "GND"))
 (segment (start 174.676 64.821) (end 178.867 69.012) (width 0.25) (layer "F.Cu") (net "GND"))
 (segment (start 141.783 90.729) (end 141.783 96.317) (width 0.25) (layer "F.Cu") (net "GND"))
 (segment (start 189.408 60.376) (end 184.963 64.821) (width 0.25) (layer "F.Cu") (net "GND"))
 (segment (start 181.788 69.012) (end 184.963 65.837) (width 0.25) (layer "F.Cu") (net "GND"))
 (segment (start 184.963 83.363) (end 193.98 92.38) (width 0.25) (layer "F.Cu") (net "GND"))
 (segment (start 178.867 69.012) (end 181.788 69.012) (width 0.25) (layer "F.Cu") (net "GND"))
 (segment (start 126.416 52.248) (end 126.416 49.2) (width 0.25) (layer "F.Cu") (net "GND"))
 (segment (start 131.369 54.153) (end 126.416 49.2) (width 0.25) (layer "F.Cu") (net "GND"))
 (segment (start 141.783 96.317) (end 140.64 97.46) (width 0.25) (layer "F.Cu") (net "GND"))
 (segment (start 184.963 64.821) (end 184.963 65.837) (width 0.25) (layer "F.Cu") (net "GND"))
 (segment (start 184.963 65.837) (end 184.963 83.363) (width 0.25) (layer "F.Cu") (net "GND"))
 (via (at 174.676 64.821) (size 0.6) (drill 0.4) (layers "F.Cu" "B.Cu") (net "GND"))
 (segment (start 153.467 54.153) (end 161.087 61.773) (width 0.25) (layer "B.Cu") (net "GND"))
 (segment (start 193.98 92.38) (end 196.52 92.38) (width 0.25) (layer "B.Cu") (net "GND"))
 (segment (start 191.821 94.539) (end 193.98 92.38) (width 0.25) (layer "B.Cu") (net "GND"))
 (segment (start 172.263 64.821) (end 174.676 64.821) (width 0.25) (layer "B.Cu") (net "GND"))
 (segment (start 143.18 97.46) (end 146.101 94.539) (width 0.25) (layer "B.Cu") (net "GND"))
 (segment (start 161.087 61.773) (end 169.215 61.773) (width 0.25) (layer "B.Cu") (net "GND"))
 (segment (start 146.101 94.539) (end 191.821 94.539) (width 0.25) (layer "B.Cu") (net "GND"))
 (segment (start 169.215 61.773) (end 172.263 64.821) (width 0.25) (layer "B.Cu") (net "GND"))
 (segment (start 140.64 97.46) (end 143.18 97.46) (width 0.25) (layer "B.Cu") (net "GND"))
 (segment (start 189.408 57.836) (end 181.407 65.837) (width 0.25) (layer "F.Cu") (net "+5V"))
 (segment (start 126.67 86.03) (end 138.1 97.46) (width 0.25) (layer "F.Cu") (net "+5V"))
 (segment (start 126.67 54.534) (end 126.67 86.03) (width 0.25) (layer "F.Cu") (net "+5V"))
 (segment (start 139.783 90.729) (end 139.783 95.777) (width 0.25) (layer "F.Cu") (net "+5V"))
 (segment (start 139.783 95.777) (end 138.1 97.46) (width 0.25) (layer "F.Cu") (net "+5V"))
 (segment (start 181.407 65.837) (end 179.963 65.837) (width 0.25) (layer "F.Cu") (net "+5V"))
 (segment (start 193.98 49.2) (end 196.52 49.2) (width 0.25) (layer "B.Cu") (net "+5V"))
 (segment (start 163.627 54.153) (end 165.786 54.153) (width 0.25) (layer "B.Cu") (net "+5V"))
 (segment (start 138.1 97.46) (end 169.723 65.837) (width 0.25) (layer "B.Cu") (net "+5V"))
 (segment (start 179.963 65.837) (end 179.963 61.846518) (width 0.25) (layer "B.Cu") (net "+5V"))
 (segment (start 175.057 60.249) (end 176.654518 61.846518) (width 0.25) (layer "B.Cu") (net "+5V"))
 (segment (start 171.882 60.249) (end 175.057 60.249) (width 0.25) (layer "B.Cu") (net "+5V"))
 (segment (start 176.517 65.837) (end 193.154 49.2) (width 0.25) (layer "B.Cu") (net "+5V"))
 (segment (start 188.704518 53.105) (end 190.075 53.105) (width 0.25) (layer "B.Cu") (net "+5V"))
 (segment (start 169.723 65.837) (end 176.517 65.837) (width 0.25) (layer "B.Cu") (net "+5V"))
 (segment (start 168.707 60.249) (end 171.882 60.249) (width 0.25) (layer "B.Cu") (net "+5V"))
 (segment (start 176.654518 61.846518) (end 179.963 61.846518) (width 0.25) (layer "B.Cu") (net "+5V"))
 (segment (start 193.154 49.2) (end 193.98 49.2) (width 0.25) (layer "B.Cu") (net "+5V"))
 (segment (start 179.963 61.846518) (end 188.704518 53.105) (width 0.25) (layer "B.Cu") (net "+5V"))
 (segment (start 161.087 54.153) (end 163.627 54.153) (width 0.25) (layer "B.Cu") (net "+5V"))
 (segment (start 165.786 54.153) (end 171.882 60.249) (width 0.25) (layer "B.Cu") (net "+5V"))
 (segment (start 168.961 54.153) (end 176.654518 61.846518) (width 0.25) (layer "B.Cu") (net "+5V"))
 (segment (start 190.075 53.105) (end 193.98 49.2) (width 0.25) (layer "B.Cu") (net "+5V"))
 (segment (start 156.007 54.153) (end 156.007 49.327) (width 0.25) (layer "F.Cu") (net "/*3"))
 (segment (start 156.007 49.327) (end 155.88 49.2) (width 0.25) (layer "F.Cu") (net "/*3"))
 (segment (start 158.547 49.327) (end 158.42 49.2) (width 0.25) (layer "F.Cu") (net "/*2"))
 (segment (start 158.547 54.153) (end 158.547 49.327) (width 0.25) (layer "F.Cu") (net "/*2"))
 (segment (start 183.185 60.249) (end 178.867 60.249) (width 0.25) (layer "F.Cu") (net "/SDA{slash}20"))
 (segment (start 121.59 49.454) (end 121.336 49.2) (width 0.25) (layer "F.Cu") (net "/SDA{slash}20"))
 (segment (start 123.749 51.613) (end 125.4 51.613) (width 0.25) (layer "F.Cu") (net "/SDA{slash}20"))
 (segment (start 121.59 54.534) (end 121.59 49.454) (width 0.25) (layer "F.Cu") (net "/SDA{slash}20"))
 (segment (start 121.336 49.2) (end 123.749 51.613) (width 0.25) (layer "F.Cu") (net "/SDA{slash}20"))
 (via (at 183.185 60.249) (size 0.6) (drill 0.4) (layers "F.Cu" "B.Cu") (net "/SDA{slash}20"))
 (via (at 125.4 51.613) (size 0.6) (drill 0.4) (layers "F.Cu" "B.Cu") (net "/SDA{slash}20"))
 (segment (start 183.82 55.296) (end 183.82 49.2) (width 0.25) (layer "B.Cu") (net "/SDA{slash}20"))
 (segment (start 178.867 60.249) (end 183.82 55.296) (width 0.25) (layer "B.Cu") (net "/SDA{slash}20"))
 (segment (start 181.407 51.613) (end 183.82 49.2) (width 0.25) (layer "B.Cu") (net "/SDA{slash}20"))
 (segment (start 186.741 60.249) (end 183.185 60.249) (width 0.25) (layer "B.Cu") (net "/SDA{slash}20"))
 (segment (start 189.408 62.916) (end 186.741 60.249) (width 0.25) (layer "B.Cu") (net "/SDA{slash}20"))
 (segment (start 125.4 51.613) (end 181.407 51.613) (width 0.25) (layer "B.Cu") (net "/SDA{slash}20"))
 (segment (start 180.518 57.709) (end 128.448 57.709) (width 0.25) (layer "F.Cu") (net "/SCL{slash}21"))
 (segment (start 179.121 54.153) (end 181.407 54.153) (width 0.25) (layer "F.Cu") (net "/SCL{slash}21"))
 (segment (start 186.233 51.994) (end 180.518 57.709) (width 0.25) (layer "F.Cu") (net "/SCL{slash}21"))
 (segment (start 119.05 54.534) (end 119.05 49.454) (width 0.25) (layer "F.Cu") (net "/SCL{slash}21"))
 (segment (start 181.407 54.153) (end 186.36 49.2) (width 0.25) (layer "F.Cu") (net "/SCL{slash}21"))
 (segment (start 189.408 52.248) (end 186.36 49.2) (width 0.25) (layer "F.Cu") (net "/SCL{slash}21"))
 (segment (start 119.05 49.454) (end 118.796 49.2) (width 0.25) (layer "F.Cu") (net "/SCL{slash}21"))
 (segment (start 189.408 55.296) (end 189.408 52.248) (width 0.25) (layer "F.Cu") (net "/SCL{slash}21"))
 (via (at 128.448 57.709) (size 0.6) (drill 0.4) (layers "F.Cu" "B.Cu") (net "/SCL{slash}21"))
 (via (at 186.233 51.994) (size 0.6) (drill 0.4) (layers "F.Cu" "B.Cu") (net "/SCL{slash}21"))
 (segment (start 122.225 57.709) (end 119.05 54.534) (width 0.25) (layer "B.Cu") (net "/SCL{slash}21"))
 (segment (start 186.36 51.867) (end 186.233 51.994) (width 0.25) (layer "B.Cu") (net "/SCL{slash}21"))
 (segment (start 128.448 57.709) (end 122.225 57.709) (width 0.25) (layer "B.Cu") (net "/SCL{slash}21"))
 (segment (start 186.36 49.2) (end 186.36 51.867) (width 0.25) (layer "B.Cu") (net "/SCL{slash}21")))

